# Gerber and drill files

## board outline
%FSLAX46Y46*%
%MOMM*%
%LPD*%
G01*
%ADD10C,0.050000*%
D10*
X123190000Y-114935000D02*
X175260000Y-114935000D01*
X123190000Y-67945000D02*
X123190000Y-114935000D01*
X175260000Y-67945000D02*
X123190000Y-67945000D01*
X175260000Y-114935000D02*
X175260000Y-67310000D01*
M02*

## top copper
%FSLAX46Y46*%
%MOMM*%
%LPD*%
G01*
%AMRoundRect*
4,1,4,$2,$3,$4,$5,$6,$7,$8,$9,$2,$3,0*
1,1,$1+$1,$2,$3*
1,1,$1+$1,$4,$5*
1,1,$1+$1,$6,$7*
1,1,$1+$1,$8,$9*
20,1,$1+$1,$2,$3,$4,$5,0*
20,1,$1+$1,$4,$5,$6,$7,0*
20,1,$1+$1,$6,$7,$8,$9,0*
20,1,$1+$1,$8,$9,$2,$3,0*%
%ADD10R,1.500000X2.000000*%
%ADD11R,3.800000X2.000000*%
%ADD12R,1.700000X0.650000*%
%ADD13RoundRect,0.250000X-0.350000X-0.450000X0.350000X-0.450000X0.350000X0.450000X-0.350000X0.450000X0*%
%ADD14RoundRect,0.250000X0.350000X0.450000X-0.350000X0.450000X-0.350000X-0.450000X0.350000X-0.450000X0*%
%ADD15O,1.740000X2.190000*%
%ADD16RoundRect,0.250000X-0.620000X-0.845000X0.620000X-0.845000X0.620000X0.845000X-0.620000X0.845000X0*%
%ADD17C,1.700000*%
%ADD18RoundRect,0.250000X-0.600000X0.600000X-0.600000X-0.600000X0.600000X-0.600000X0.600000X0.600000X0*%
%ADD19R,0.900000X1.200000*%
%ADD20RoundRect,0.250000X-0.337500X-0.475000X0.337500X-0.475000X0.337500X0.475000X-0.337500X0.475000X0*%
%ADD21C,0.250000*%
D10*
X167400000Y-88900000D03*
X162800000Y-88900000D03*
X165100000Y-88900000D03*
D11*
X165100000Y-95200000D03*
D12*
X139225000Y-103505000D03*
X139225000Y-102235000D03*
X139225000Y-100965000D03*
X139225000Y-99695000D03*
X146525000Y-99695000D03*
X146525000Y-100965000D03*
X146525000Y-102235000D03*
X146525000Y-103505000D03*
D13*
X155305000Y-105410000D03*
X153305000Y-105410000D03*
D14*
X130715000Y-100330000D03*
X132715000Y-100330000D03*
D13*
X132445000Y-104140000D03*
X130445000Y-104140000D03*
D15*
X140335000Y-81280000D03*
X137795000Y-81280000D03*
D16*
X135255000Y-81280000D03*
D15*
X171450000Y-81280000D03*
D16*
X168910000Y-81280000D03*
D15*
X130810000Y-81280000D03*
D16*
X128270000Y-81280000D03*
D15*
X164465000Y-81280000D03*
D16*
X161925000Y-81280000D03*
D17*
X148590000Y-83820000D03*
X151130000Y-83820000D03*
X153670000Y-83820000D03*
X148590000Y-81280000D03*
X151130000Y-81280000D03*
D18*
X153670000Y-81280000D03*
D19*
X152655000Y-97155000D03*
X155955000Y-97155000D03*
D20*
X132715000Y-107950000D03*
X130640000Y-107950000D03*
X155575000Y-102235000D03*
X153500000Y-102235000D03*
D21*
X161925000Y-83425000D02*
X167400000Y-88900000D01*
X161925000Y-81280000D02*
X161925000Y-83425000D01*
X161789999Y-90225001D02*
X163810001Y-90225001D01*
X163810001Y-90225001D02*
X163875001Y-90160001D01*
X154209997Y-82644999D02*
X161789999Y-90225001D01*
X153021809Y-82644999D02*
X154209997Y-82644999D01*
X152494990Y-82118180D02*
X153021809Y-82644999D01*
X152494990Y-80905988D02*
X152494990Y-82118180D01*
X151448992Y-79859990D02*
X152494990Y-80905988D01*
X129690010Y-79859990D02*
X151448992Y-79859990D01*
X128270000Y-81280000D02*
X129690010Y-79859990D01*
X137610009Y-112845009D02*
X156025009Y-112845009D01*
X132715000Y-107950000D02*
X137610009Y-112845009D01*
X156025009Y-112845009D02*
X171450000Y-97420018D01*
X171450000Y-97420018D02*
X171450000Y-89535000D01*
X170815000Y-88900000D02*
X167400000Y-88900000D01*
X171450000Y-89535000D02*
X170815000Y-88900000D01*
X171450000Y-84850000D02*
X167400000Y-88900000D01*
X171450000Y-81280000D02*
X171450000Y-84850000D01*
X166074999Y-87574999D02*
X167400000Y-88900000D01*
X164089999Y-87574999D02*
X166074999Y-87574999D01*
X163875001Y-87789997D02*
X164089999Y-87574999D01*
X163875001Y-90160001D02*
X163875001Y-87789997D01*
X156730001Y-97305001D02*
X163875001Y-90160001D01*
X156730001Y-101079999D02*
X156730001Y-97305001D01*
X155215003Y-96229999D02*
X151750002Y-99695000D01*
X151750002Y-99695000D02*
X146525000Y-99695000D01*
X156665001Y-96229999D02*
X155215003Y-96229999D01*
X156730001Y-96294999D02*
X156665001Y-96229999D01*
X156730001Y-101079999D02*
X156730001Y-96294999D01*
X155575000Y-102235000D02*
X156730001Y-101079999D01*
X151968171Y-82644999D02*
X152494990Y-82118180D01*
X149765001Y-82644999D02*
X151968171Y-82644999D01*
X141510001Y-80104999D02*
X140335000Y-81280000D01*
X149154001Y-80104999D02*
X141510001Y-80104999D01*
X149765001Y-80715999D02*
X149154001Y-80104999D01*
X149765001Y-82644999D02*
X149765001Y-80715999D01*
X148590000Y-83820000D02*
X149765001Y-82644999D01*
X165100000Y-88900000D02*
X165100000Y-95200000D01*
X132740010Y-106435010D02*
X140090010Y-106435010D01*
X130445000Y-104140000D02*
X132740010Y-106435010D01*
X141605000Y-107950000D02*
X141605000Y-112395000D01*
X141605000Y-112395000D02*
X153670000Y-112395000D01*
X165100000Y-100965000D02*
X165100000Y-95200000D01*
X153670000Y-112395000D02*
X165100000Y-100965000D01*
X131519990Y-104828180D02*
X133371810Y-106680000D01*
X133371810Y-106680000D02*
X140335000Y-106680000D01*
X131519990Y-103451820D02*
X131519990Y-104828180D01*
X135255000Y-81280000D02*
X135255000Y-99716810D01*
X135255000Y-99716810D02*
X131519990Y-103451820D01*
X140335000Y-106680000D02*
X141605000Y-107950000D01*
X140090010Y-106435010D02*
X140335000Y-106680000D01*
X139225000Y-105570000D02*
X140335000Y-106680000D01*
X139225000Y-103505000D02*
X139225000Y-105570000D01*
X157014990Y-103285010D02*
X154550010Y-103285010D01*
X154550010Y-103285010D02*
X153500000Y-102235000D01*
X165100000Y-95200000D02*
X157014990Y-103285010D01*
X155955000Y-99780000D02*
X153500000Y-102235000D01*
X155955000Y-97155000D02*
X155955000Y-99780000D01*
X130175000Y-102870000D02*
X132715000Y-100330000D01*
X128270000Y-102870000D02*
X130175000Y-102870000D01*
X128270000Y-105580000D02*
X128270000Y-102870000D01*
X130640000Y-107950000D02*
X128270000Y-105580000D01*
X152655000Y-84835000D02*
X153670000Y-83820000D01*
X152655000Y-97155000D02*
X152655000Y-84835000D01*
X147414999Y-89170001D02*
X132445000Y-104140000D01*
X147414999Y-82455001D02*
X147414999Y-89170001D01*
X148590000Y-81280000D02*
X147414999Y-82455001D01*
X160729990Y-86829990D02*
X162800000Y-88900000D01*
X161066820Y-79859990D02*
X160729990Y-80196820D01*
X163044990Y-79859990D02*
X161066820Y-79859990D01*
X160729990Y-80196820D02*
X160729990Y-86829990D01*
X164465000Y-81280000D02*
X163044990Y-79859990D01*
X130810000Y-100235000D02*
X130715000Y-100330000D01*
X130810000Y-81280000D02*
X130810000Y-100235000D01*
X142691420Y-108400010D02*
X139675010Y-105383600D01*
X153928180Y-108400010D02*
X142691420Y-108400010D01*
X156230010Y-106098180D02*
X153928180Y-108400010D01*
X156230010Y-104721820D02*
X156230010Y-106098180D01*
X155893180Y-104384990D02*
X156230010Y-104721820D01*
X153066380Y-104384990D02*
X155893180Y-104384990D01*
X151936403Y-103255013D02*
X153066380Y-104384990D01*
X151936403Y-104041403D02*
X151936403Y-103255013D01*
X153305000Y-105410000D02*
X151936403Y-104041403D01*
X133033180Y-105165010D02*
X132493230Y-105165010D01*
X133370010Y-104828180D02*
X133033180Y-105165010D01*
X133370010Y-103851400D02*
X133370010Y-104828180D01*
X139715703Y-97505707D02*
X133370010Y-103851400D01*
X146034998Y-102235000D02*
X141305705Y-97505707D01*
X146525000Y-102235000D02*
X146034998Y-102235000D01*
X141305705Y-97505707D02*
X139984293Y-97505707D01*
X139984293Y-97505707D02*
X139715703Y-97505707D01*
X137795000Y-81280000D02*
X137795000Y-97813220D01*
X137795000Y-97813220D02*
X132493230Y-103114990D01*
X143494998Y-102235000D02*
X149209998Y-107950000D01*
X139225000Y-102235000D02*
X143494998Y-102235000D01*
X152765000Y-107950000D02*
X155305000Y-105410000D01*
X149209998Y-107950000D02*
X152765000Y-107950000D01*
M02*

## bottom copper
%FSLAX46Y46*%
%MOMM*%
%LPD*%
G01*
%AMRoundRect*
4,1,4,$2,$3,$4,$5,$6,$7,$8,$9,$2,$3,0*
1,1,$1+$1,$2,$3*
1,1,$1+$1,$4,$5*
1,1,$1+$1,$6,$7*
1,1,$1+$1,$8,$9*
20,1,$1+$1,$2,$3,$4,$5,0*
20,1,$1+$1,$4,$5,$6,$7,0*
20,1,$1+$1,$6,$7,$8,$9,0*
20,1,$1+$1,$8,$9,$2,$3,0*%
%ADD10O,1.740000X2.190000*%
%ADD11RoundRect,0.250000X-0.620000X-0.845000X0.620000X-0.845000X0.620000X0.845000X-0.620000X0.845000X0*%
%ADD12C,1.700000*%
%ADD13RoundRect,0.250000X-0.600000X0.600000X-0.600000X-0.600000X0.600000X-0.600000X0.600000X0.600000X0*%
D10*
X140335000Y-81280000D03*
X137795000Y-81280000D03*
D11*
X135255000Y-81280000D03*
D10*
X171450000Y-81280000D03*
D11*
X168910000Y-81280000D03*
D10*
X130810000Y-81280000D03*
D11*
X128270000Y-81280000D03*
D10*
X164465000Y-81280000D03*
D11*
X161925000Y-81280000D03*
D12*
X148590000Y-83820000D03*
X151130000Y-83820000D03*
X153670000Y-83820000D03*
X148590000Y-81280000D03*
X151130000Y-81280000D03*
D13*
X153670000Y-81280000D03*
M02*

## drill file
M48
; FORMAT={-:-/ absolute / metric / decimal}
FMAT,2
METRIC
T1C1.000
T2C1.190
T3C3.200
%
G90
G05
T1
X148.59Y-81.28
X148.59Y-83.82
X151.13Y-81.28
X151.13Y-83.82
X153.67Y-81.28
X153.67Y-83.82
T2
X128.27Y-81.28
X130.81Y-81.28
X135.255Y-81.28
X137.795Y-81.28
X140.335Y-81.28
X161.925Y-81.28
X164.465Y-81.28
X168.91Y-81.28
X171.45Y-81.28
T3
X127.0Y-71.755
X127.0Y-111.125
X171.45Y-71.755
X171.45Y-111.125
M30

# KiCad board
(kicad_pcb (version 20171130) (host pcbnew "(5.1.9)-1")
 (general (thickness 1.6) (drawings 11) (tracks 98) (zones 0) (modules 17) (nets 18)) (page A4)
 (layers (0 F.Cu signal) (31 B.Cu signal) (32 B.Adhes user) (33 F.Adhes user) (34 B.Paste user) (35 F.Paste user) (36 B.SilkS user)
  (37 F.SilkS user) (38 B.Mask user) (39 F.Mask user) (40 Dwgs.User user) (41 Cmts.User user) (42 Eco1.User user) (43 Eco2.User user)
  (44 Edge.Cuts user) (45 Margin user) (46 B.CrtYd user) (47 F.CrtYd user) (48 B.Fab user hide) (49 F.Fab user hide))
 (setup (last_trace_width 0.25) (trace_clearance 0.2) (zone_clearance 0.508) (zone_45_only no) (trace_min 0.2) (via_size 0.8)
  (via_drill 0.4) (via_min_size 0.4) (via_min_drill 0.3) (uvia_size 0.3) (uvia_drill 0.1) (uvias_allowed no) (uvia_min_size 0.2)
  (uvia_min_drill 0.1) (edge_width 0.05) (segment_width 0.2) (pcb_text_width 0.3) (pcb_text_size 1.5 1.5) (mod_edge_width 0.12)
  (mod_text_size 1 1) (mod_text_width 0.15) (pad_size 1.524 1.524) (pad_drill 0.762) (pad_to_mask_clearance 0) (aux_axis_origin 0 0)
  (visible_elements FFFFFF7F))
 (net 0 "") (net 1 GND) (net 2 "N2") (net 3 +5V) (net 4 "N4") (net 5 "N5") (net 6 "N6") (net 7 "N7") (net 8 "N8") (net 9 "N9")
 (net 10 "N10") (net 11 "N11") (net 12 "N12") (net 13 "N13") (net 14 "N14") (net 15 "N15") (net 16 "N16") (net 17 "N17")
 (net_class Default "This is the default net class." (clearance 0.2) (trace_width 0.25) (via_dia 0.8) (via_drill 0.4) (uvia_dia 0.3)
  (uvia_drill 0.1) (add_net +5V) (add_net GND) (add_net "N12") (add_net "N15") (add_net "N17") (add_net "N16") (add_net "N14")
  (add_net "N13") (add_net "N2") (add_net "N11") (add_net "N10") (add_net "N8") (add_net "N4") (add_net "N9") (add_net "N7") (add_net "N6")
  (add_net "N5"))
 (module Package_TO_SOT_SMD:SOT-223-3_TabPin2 (layer F.Cu) (at 165.1 92.05 270)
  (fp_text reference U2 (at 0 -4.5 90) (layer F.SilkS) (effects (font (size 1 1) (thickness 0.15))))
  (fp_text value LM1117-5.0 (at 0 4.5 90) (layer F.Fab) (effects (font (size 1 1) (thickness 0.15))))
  (pad 1 smd rect (at -3.15 -2.3 270) (size 2 1.5) (layers F.Cu F.Paste F.Mask) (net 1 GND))
  (pad 3 smd rect (at -3.15 2.3 270) (size 2 1.5) (layers F.Cu F.Paste F.Mask) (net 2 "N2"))
  (pad 2 smd rect (at -3.15 0 270) (size 2 1.5) (layers F.Cu F.Paste F.Mask) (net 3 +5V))
  (pad 2 smd rect (at 3.15 0 270) (size 2 3.8) (layers F.Cu F.Paste F.Mask) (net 3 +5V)))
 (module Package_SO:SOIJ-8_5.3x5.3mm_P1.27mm (layer F.Cu) (at 142.875 101.6 180)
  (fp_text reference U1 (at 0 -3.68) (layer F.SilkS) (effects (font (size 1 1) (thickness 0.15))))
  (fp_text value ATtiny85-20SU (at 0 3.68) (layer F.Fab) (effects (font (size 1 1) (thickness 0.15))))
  (pad 8 smd rect (at 3.65 -1.905 180) (size 1.7 0.65) (layers F.Cu F.Paste F.Mask) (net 3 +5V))
  (pad 7 smd rect (at 3.65 -0.635 180) (size 1.7 0.65) (layers F.Cu F.Paste F.Mask) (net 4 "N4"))
  (pad 6 smd rect (at 3.65 0.635 180) (size 1.7 0.65) (layers F.Cu F.Paste F.Mask) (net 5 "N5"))
  (pad 5 smd rect (at 3.65 1.905 180) (size 1.7 0.65) (layers F.Cu F.Paste F.Mask) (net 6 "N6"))
  (pad 4 smd rect (at -3.65 1.905 180) (size 1.7 0.65) (layers F.Cu F.Paste F.Mask) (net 1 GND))
  (pad 3 smd rect (at -3.65 0.635 180) (size 1.7 0.65) (layers F.Cu F.Paste F.Mask) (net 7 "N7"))
  (pad 2 smd rect (at -3.65 -0.635 180) (size 1.7 0.65) (layers F.Cu F.Paste F.Mask) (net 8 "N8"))
  (pad 1 smd rect (at -3.65 -1.905 180) (size 1.7 0.65) (layers F.Cu F.Paste F.Mask) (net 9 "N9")))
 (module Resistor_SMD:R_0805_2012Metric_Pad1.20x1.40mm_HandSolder (layer F.Cu) (at 154.305 105.41)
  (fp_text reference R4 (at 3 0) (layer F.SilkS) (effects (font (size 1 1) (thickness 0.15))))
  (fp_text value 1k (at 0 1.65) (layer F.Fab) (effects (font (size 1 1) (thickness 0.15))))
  (pad 2 smd roundrect (at 1 0) (size 1.2 1.4) (layers F.Cu F.Paste F.Mask) (roundrect_rratio 0.208333) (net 4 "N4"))
  (pad 1 smd roundrect (at -1 0) (size 1.2 1.4) (layers F.Cu F.Paste F.Mask) (roundrect_rratio 0.208333) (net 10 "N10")))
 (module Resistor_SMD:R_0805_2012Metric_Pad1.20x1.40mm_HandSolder (layer F.Cu) (at 131.715 100.33 180)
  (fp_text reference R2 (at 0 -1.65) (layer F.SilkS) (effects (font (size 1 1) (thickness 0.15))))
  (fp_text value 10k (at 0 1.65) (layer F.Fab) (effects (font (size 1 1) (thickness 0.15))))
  (pad 2 smd roundrect (at 1 0 180) (size 1.2 1.4) (layers F.Cu F.Paste F.Mask) (roundrect_rratio 0.208333) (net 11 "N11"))
  (pad 1 smd roundrect (at -1 0 180) (size 1.2 1.4) (layers F.Cu F.Paste F.Mask) (roundrect_rratio 0.208333) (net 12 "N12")))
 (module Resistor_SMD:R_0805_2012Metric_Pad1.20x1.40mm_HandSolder (layer F.Cu) (at 131.445 104.14)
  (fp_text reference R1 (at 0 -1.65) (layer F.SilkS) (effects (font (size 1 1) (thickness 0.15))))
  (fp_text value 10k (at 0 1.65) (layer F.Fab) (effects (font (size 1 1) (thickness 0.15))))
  (pad 2 smd roundrect (at 1 0) (size 1.2 1.4) (layers F.Cu F.Paste F.Mask) (roundrect_rratio 0.208333) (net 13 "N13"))
  (pad 1 smd roundrect (at -1 0) (size 1.2 1.4) (layers F.Cu F.Paste F.Mask) (roundrect_rratio 0.208333) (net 3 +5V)))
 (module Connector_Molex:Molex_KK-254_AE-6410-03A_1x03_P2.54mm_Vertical (layer F.Cu) (at 135.255 81.28)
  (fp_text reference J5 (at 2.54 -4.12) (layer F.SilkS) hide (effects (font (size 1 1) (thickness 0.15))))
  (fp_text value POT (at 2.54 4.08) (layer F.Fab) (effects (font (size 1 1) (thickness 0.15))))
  (pad 3 thru_hole oval (at 5.08 0) (size 1.74 2.19) (drill 1.19) (layers *.Cu *.Mask) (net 1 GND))
  (pad 2 thru_hole oval (at 2.54 0) (size 1.74 2.19) (drill 1.19) (layers *.Cu *.Mask) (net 8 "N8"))
  (pad 1 thru_hole roundrect (at 0 0) (size 1.74 2.19) (drill 1.19) (layers *.Cu *.Mask) (roundrect_rratio 0.143678) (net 3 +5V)))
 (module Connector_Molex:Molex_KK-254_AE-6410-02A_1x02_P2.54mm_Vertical (layer F.Cu) (at 168.91 81.28)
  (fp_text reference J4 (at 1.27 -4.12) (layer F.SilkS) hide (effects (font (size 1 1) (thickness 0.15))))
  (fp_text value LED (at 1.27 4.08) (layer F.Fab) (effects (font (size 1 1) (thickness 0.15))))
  (pad 2 thru_hole oval (at 2.54 0) (size 1.74 2.19) (drill 1.19) (layers *.Cu *.Mask) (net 1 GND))
  (pad 1 thru_hole roundrect (at 0 0) (size 1.74 2.19) (drill 1.19) (layers *.Cu *.Mask) (roundrect_rratio 0.143678) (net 10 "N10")))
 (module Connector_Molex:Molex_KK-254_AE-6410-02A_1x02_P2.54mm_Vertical (layer F.Cu) (at 128.27 81.28)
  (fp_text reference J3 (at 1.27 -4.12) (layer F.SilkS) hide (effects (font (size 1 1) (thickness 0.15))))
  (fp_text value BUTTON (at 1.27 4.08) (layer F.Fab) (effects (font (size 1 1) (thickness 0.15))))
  (pad 2 thru_hole oval (at 2.54 0) (size 1.74 2.19) (drill 1.19) (layers *.Cu *.Mask) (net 11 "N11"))
  (pad 1 thru_hole roundrect (at 0 0) (size 1.74 2.19) (drill 1.19) (layers *.Cu *.Mask) (roundrect_rratio 0.143678) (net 1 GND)))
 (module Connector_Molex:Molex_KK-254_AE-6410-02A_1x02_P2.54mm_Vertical (layer F.Cu) (at 161.925 81.28)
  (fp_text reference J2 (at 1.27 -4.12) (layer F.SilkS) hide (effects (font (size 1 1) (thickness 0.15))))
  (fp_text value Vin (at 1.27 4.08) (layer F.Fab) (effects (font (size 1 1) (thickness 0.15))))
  (pad 2 thru_hole oval (at 2.54 0) (size 1.74 2.19) (drill 1.19) (layers *.Cu *.Mask) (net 2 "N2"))
  (pad 1 thru_hole roundrect (at 0 0) (size 1.74 2.19) (drill 1.19) (layers *.Cu *.Mask) (roundrect_rratio 0.143678) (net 1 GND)))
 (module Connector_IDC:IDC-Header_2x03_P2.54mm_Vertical (layer F.Cu) (at 153.67 81.28 270)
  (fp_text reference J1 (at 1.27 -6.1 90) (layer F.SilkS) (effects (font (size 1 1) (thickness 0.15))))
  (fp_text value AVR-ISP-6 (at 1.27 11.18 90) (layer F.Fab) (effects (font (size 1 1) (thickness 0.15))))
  (pad 6 thru_hole circle (at 2.54 5.08 270) (size 1.7 1.7) (drill 1) (layers *.Cu *.Mask) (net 1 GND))
  (pad 4 thru_hole circle (at 2.54 2.54 270) (size 1.7 1.7) (drill 1) (layers *.Cu *.Mask) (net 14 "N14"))
  (pad 2 thru_hole circle (at 2.54 0 270) (size 1.7 1.7) (drill 1) (layers *.Cu *.Mask) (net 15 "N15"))
  (pad 5 thru_hole circle (at 0 5.08 270) (size 1.7 1.7) (drill 1) (layers *.Cu *.Mask) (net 13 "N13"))
  (pad 3 thru_hole circle (at 0 2.54 270) (size 1.7 1.7) (drill 1) (layers *.Cu *.Mask) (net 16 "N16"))
  (pad 1 thru_hole roundrect (at 0 0 270) (size 1.7 1.7) (drill 1) (layers *.Cu *.Mask) (roundrect_rratio 0.147059) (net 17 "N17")))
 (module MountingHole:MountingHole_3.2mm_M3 (layer F.Cu) (at 127 111.125)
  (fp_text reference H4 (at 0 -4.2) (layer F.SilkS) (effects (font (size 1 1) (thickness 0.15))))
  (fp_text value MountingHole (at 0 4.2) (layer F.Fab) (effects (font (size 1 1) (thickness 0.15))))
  (pad 1 np_thru_hole circle (at 0 0) (size 3.2 3.2) (drill 3.2) (layers *.Cu *.Mask)))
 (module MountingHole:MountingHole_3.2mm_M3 (layer F.Cu) (at 171.45 71.755)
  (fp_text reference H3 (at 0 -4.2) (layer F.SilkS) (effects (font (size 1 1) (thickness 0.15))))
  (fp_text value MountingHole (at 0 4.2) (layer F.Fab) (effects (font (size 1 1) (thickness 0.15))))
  (pad 1 np_thru_hole circle (at 0 0) (size 3.2 3.2) (drill 3.2) (layers *.Cu *.Mask)))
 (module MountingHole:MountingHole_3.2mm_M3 (layer F.Cu) (at 127 71.755)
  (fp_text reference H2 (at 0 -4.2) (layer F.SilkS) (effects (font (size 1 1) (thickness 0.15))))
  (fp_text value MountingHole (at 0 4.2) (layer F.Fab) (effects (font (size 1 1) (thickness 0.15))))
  (pad 1 np_thru_hole circle (at 0 0) (size 3.2 3.2) (drill 3.2) (layers *.Cu *.Mask)))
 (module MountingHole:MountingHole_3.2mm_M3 (layer F.Cu) (at 171.45 111.125)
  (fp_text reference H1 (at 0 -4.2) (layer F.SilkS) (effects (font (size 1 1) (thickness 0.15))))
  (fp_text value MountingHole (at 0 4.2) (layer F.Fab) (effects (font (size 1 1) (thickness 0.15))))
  (pad 1 np_thru_hole circle (at 0 0) (size 3.2 3.2) (drill 3.2) (layers *.Cu *.Mask)))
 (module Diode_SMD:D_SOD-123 (layer F.Cu) (at 154.305 97.155 180)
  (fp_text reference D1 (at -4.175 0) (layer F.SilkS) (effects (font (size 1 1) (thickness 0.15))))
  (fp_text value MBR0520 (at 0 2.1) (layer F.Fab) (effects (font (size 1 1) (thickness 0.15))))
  (pad 2 smd rect (at 1.65 0 180) (size 0.9 1.2) (layers F.Cu F.Paste F.Mask) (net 15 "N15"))
  (pad 1 smd rect (at -1.65 0 180) (size 0.9 1.2) (layers F.Cu F.Paste F.Mask) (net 3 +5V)))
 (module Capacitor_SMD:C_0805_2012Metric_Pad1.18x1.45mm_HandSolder (layer F.Cu) (at 131.6775 107.95)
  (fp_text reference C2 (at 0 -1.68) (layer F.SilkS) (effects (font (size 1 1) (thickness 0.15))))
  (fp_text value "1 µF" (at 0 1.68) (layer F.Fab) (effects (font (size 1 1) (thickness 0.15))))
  (pad 2 smd roundrect (at 1.0375 0) (size 1.175 1.45) (layers F.Cu F.Paste F.Mask) (roundrect_rratio 0.212766) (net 1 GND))
  (pad 1 smd roundrect (at -1.0375 0) (size 1.175 1.45) (layers F.Cu F.Paste F.Mask) (roundrect_rratio 0.212766) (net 12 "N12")))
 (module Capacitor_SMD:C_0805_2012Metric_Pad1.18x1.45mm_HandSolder (layer F.Cu) (at 154.5375 102.235)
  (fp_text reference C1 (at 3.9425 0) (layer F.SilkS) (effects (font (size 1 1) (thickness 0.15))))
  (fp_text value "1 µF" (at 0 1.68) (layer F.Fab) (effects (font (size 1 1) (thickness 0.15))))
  (pad 2 smd roundrect (at 1.0375 0) (size 1.175 1.45) (layers F.Cu F.Paste F.Mask) (roundrect_rratio 0.212766) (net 1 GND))
  (pad 1 smd roundrect (at -1.0375 0) (size 1.175 1.45) (layers F.Cu F.Paste F.Mask) (roundrect_rratio 0.212766) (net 3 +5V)))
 (gr_line (start 123.19 114.935) (end 175.26 114.935) (layer Edge.Cuts) (width 0.05))
 (gr_line (start 123.19 67.945) (end 123.19 114.935) (layer Edge.Cuts) (width 0.05))
 (gr_line (start 175.26 67.945) (end 123.19 67.945) (layer Edge.Cuts) (width 0.05))
 (gr_line (start 175.26 114.935) (end 175.26 67.31) (layer Edge.Cuts) (width 0.05))
 (segment (start 161.925 83.425) (end 167.4 88.9) (width 0.25) (layer F.Cu) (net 1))
 (segment (start 161.925 81.28) (end 161.925 83.425) (width 0.25) (layer F.Cu) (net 1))
 (segment (start 161.789999 90.225001) (end 163.810001 90.225001) (width 0.25) (layer F.Cu) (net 1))
 (segment (start 163.810001 90.225001) (end 163.875001 90.160001) (width 0.25) (layer F.Cu) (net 1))
 (segment (start 154.209997 82.644999) (end 161.789999 90.225001) (width 0.25) (layer F.Cu) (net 1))
 (segment (start 153.021809 82.644999) (end 154.209997 82.644999) (width 0.25) (layer F.Cu) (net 1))
 (segment (start 152.49499 82.11818) (end 153.021809 82.644999) (width 0.25) (layer F.Cu) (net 1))
 (segment (start 152.49499 80.905988) (end 152.49499 82.11818) (width 0.25) (layer F.Cu) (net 1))
 (segment (start 151.448992 79.85999) (end 152.49499 80.905988) (width 0.25) (layer F.Cu) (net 1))
 (segment (start 129.69001 79.85999) (end 151.448992 79.85999) (width 0.25) (layer F.Cu) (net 1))
 (segment (start 128.27 81.28) (end 129.69001 79.85999) (width 0.25) (layer F.Cu) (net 1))
 (segment (start 137.610009 112.845009) (end 156.025009 112.845009) (width 0.25) (layer F.Cu) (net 1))
 (segment (start 132.715 107.95) (end 137.610009 112.845009) (width 0.25) (layer F.Cu) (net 1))
 (segment (start 156.025009 112.845009) (end 171.45 97.420018) (width 0.25) (layer F.Cu) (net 1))
 (segment (start 171.45 97.420018) (end 171.45 89.535) (width 0.25) (layer F.Cu) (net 1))
 (segment (start 170.815 88.9) (end 167.4 88.9) (width 0.25) (layer F.Cu) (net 1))
 (segment (start 171.45 89.535) (end 170.815 88.9) (width 0.25) (layer F.Cu) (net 1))
 (segment (start 171.45 84.85) (end 167.4 88.9) (width 0.25) (layer F.Cu) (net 1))
 (segment (start 171.45 81.28) (end 171.45 84.85) (width 0.25) (layer F.Cu) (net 1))
 (segment (start 166.074999 87.574999) (end 167.4 88.9) (width 0.25) (layer F.Cu) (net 1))
 (segment (start 164.089999 87.574999) (end 166.074999 87.574999) (width 0.25) (layer F.Cu) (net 1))
 (segment (start 163.875001 87.789997) (end 164.089999 87.574999) (width 0.25) (layer F.Cu) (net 1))
 (segment (start 163.875001 90.160001) (end 163.875001 87.789997) (width 0.25) (layer F.Cu) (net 1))
 (segment (start 156.730001 97.305001) (end 163.875001 90.160001) (width 0.25) (layer F.Cu) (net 1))
 (segment (start 156.730001 101.079999) (end 156.730001 97.305001) (width 0.25) (layer F.Cu) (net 1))
 (segment (start 155.215003 96.229999) (end 151.750002 99.695) (width 0.25) (layer F.Cu) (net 1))
 (segment (start 151.750002 99.695) (end 146.525 99.695) (width 0.25) (layer F.Cu) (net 1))
 (segment (start 156.665001 96.229999) (end 155.215003 96.229999) (width 0.25) (layer F.Cu) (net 1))
 (segment (start 156.730001 96.294999) (end 156.665001 96.229999) (width 0.25) (layer F.Cu) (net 1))
 (segment (start 156.730001 101.079999) (end 156.730001 96.294999) (width 0.25) (layer F.Cu) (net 1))
 (segment (start 155.575 102.235) (end 156.730001 101.079999) (width 0.25) (layer F.Cu) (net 1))
 (segment (start 151.968171 82.644999) (end 152.49499 82.11818) (width 0.25) (layer F.Cu) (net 1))
 (segment (start 149.765001 82.644999) (end 151.968171 82.644999) (width 0.25) (layer F.Cu) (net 1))
 (segment (start 141.510001 80.104999) (end 140.335 81.28) (width 0.25) (layer F.Cu) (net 1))
 (segment (start 149.154001 80.104999) (end 141.510001 80.104999) (width 0.25) (layer F.Cu) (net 1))
 (segment (start 149.765001 80.715999) (end 149.154001 80.104999) (width 0.25) (layer F.Cu) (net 1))
 (segment (start 149.765001 82.644999) (end 149.765001 80.715999) (width 0.25) (layer F.Cu) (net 1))
 (segment (start 148.59 83.82) (end 149.765001 82.644999) (width 0.25) (layer F.Cu) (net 1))
 (segment (start 165.1 88.9) (end 165.1 95.2) (width 0.25) (layer F.Cu) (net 3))
 (segment (start 132.74001 106.43501) (end 140.09001 106.43501) (width 0.25) (layer F.Cu) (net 3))
 (segment (start 130.445 104.14) (end 132.74001 106.43501) (width 0.25) (layer F.Cu) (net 3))
 (segment (start 141.605 107.95) (end 141.605 112.395) (width 0.25) (layer F.Cu) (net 3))
 (segment (start 141.605 112.395) (end 153.67 112.395) (width 0.25) (layer F.Cu) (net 3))
 (segment (start 165.1 100.965) (end 165.1 95.2) (width 0.25) (layer F.Cu) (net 3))
 (segment (start 153.67 112.395) (end 165.1 100.965) (width 0.25) (layer F.Cu) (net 3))
 (segment (start 131.51999 104.82818) (end 133.37181 106.68) (width 0.25) (layer F.Cu) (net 3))
 (segment (start 133.37181 106.68) (end 140.335 106.68) (width 0.25) (layer F.Cu) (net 3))
 (segment (start 131.51999 103.45182) (end 131.51999 104.82818) (width 0.25) (layer F.Cu) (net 3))
 (segment (start 135.255 81.28) (end 135.255 99.71681) (width 0.25) (layer F.Cu) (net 3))
 (segment (start 135.255 99.71681) (end 131.51999 103.45182) (width 0.25) (layer F.Cu) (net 3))
 (segment (start 140.335 106.68) (end 141.605 107.95) (width 0.25) (layer F.Cu) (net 3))
 (segment (start 140.09001 106.43501) (end 140.335 106.68) (width 0.25) (layer F.Cu) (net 3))
 (segment (start 139.225 105.57) (end 140.335 106.68) (width 0.25) (layer F.Cu) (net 3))
 (segment (start 139.225 103.505) (end 139.225 105.57) (width 0.25) (layer F.Cu) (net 3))
 (segment (start 157.01499 103.28501) (end 154.55001 103.28501) (width 0.25) (layer F.Cu) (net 3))
 (segment (start 154.55001 103.28501) (end 153.5 102.235) (width 0.25) (layer F.Cu) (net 3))
 (segment (start 165.1 95.2) (end 157.01499 103.28501) (width 0.25) (layer F.Cu) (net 3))
 (segment (start 155.955 99.78) (end 153.5 102.235) (width 0.25) (layer F.Cu) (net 3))
 (segment (start 155.955 97.155) (end 155.955 99.78) (width 0.25) (layer F.Cu) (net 3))
 (segment (start 130.175 102.87) (end 132.715 100.33) (width 0.25) (layer F.Cu) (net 12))
 (segment (start 128.27 102.87) (end 130.175 102.87) (width 0.25) (layer F.Cu) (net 12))
 (segment (start 128.27 105.58) (end 128.27 102.87) (width 0.25) (layer F.Cu) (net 12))
 (segment (start 130.64 107.95) (end 128.27 105.58) (width 0.25) (layer F.Cu) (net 12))
 (segment (start 152.655 84.835) (end 153.67 83.82) (width 0.25) (layer F.Cu) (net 15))
 (segment (start 152.655 97.155) (end 152.655 84.835) (width 0.25) (layer F.Cu) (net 15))
 (segment (start 147.414999 89.170001) (end 132.445 104.14) (width 0.25) (layer F.Cu) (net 13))
 (segment (start 147.414999 82.455001) (end 147.414999 89.170001) (width 0.25) (layer F.Cu) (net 13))
 (segment (start 148.59 81.28) (end 147.414999 82.455001) (width 0.25) (layer F.Cu) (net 13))
 (segment (start 160.72999 86.82999) (end 162.8 88.9) (width 0.25) (layer F.Cu) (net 2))
 (segment (start 161.06682 79.85999) (end 160.72999 80.19682) (width 0.25) (layer F.Cu) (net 2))
 (segment (start 163.04499 79.85999) (end 161.06682 79.85999) (width 0.25) (layer F.Cu) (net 2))
 (segment (start 160.72999 80.19682) (end 160.72999 86.82999) (width 0.25) (layer F.Cu) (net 2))
 (segment (start 164.465 81.28) (end 163.04499 79.85999) (width 0.25) (layer F.Cu) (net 2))
 (segment (start 130.81 100.235) (end 130.715 100.33) (width 0.25) (layer F.Cu) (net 11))
 (segment (start 130.81 81.28) (end 130.81 100.235) (width 0.25) (layer F.Cu) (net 11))
 (segment (start 142.69142 108.40001) (end 139.67501 105.3836) (width 0.25) (layer F.Cu) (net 10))
 (segment (start 153.92818 108.40001) (end 142.69142 108.40001) (width 0.25) (layer F.Cu) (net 10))
 (segment (start 156.23001 106.09818) (end 153.92818 108.40001) (width 0.25) (layer F.Cu) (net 10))
 (segment (start 156.23001 104.72182) (end 156.23001 106.09818) (width 0.25) (layer F.Cu) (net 10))
 (segment (start 155.89318 104.38499) (end 156.23001 104.72182) (width 0.25) (layer F.Cu) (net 10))
 (segment (start 153.06638 104.38499) (end 155.89318 104.38499) (width 0.25) (layer F.Cu) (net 10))
 (segment (start 151.936403 103.255013) (end 153.06638 104.38499) (width 0.25) (layer F.Cu) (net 10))
 (segment (start 151.936403 104.041403) (end 151.936403 103.255013) (width 0.25) (layer F.Cu) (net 10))
 (segment (start 153.305 105.41) (end 151.936403 104.041403) (width 0.25) (layer F.Cu) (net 10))
 (segment (start 133.03318 105.16501) (end 132.49323 105.16501) (width 0.25) (layer F.Cu) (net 8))
 (segment (start 133.37001 104.82818) (end 133.03318 105.16501) (width 0.25) (layer F.Cu) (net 8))
 (segment (start 133.37001 103.8514) (end 133.37001 104.82818) (width 0.25) (layer F.Cu) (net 8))
 (segment (start 139.715703 97.505707) (end 133.37001 103.8514) (width 0.25) (layer F.Cu) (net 8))
 (segment (start 146.034998 102.235) (end 141.305705 97.505707) (width 0.25) (layer F.Cu) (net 8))
 (segment (start 146.525 102.235) (end 146.034998 102.235) (width 0.25) (layer F.Cu) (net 8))
 (segment (start 141.305705 97.505707) (end 139.984293 97.505707) (width 0.25) (layer F.Cu) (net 8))
 (segment (start 139.984293 97.505707) (end 139.715703 97.505707) (width 0.25) (layer F.Cu) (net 8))
 (segment (start 137.795 81.28) (end 137.795 97.81322) (width 0.25) (layer F.Cu) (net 8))
 (segment (start 137.795 97.81322) (end 132.49323 103.11499) (width 0.25) (layer F.Cu) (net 8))
 (segment (start 143.494998 102.235) (end 149.209998 107.95) (width 0.25) (layer F.Cu) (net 4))
 (segment (start 139.225 102.235) (end 143.494998 102.235) (width 0.25) (layer F.Cu) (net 4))
 (segment (start 152.765 107.95) (end 155.305 105.41) (width 0.25) (layer F.Cu) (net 4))
 (segment (start 149.209998 107.95) (end 152.765 107.95) (width 0.25) (layer F.Cu) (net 4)))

